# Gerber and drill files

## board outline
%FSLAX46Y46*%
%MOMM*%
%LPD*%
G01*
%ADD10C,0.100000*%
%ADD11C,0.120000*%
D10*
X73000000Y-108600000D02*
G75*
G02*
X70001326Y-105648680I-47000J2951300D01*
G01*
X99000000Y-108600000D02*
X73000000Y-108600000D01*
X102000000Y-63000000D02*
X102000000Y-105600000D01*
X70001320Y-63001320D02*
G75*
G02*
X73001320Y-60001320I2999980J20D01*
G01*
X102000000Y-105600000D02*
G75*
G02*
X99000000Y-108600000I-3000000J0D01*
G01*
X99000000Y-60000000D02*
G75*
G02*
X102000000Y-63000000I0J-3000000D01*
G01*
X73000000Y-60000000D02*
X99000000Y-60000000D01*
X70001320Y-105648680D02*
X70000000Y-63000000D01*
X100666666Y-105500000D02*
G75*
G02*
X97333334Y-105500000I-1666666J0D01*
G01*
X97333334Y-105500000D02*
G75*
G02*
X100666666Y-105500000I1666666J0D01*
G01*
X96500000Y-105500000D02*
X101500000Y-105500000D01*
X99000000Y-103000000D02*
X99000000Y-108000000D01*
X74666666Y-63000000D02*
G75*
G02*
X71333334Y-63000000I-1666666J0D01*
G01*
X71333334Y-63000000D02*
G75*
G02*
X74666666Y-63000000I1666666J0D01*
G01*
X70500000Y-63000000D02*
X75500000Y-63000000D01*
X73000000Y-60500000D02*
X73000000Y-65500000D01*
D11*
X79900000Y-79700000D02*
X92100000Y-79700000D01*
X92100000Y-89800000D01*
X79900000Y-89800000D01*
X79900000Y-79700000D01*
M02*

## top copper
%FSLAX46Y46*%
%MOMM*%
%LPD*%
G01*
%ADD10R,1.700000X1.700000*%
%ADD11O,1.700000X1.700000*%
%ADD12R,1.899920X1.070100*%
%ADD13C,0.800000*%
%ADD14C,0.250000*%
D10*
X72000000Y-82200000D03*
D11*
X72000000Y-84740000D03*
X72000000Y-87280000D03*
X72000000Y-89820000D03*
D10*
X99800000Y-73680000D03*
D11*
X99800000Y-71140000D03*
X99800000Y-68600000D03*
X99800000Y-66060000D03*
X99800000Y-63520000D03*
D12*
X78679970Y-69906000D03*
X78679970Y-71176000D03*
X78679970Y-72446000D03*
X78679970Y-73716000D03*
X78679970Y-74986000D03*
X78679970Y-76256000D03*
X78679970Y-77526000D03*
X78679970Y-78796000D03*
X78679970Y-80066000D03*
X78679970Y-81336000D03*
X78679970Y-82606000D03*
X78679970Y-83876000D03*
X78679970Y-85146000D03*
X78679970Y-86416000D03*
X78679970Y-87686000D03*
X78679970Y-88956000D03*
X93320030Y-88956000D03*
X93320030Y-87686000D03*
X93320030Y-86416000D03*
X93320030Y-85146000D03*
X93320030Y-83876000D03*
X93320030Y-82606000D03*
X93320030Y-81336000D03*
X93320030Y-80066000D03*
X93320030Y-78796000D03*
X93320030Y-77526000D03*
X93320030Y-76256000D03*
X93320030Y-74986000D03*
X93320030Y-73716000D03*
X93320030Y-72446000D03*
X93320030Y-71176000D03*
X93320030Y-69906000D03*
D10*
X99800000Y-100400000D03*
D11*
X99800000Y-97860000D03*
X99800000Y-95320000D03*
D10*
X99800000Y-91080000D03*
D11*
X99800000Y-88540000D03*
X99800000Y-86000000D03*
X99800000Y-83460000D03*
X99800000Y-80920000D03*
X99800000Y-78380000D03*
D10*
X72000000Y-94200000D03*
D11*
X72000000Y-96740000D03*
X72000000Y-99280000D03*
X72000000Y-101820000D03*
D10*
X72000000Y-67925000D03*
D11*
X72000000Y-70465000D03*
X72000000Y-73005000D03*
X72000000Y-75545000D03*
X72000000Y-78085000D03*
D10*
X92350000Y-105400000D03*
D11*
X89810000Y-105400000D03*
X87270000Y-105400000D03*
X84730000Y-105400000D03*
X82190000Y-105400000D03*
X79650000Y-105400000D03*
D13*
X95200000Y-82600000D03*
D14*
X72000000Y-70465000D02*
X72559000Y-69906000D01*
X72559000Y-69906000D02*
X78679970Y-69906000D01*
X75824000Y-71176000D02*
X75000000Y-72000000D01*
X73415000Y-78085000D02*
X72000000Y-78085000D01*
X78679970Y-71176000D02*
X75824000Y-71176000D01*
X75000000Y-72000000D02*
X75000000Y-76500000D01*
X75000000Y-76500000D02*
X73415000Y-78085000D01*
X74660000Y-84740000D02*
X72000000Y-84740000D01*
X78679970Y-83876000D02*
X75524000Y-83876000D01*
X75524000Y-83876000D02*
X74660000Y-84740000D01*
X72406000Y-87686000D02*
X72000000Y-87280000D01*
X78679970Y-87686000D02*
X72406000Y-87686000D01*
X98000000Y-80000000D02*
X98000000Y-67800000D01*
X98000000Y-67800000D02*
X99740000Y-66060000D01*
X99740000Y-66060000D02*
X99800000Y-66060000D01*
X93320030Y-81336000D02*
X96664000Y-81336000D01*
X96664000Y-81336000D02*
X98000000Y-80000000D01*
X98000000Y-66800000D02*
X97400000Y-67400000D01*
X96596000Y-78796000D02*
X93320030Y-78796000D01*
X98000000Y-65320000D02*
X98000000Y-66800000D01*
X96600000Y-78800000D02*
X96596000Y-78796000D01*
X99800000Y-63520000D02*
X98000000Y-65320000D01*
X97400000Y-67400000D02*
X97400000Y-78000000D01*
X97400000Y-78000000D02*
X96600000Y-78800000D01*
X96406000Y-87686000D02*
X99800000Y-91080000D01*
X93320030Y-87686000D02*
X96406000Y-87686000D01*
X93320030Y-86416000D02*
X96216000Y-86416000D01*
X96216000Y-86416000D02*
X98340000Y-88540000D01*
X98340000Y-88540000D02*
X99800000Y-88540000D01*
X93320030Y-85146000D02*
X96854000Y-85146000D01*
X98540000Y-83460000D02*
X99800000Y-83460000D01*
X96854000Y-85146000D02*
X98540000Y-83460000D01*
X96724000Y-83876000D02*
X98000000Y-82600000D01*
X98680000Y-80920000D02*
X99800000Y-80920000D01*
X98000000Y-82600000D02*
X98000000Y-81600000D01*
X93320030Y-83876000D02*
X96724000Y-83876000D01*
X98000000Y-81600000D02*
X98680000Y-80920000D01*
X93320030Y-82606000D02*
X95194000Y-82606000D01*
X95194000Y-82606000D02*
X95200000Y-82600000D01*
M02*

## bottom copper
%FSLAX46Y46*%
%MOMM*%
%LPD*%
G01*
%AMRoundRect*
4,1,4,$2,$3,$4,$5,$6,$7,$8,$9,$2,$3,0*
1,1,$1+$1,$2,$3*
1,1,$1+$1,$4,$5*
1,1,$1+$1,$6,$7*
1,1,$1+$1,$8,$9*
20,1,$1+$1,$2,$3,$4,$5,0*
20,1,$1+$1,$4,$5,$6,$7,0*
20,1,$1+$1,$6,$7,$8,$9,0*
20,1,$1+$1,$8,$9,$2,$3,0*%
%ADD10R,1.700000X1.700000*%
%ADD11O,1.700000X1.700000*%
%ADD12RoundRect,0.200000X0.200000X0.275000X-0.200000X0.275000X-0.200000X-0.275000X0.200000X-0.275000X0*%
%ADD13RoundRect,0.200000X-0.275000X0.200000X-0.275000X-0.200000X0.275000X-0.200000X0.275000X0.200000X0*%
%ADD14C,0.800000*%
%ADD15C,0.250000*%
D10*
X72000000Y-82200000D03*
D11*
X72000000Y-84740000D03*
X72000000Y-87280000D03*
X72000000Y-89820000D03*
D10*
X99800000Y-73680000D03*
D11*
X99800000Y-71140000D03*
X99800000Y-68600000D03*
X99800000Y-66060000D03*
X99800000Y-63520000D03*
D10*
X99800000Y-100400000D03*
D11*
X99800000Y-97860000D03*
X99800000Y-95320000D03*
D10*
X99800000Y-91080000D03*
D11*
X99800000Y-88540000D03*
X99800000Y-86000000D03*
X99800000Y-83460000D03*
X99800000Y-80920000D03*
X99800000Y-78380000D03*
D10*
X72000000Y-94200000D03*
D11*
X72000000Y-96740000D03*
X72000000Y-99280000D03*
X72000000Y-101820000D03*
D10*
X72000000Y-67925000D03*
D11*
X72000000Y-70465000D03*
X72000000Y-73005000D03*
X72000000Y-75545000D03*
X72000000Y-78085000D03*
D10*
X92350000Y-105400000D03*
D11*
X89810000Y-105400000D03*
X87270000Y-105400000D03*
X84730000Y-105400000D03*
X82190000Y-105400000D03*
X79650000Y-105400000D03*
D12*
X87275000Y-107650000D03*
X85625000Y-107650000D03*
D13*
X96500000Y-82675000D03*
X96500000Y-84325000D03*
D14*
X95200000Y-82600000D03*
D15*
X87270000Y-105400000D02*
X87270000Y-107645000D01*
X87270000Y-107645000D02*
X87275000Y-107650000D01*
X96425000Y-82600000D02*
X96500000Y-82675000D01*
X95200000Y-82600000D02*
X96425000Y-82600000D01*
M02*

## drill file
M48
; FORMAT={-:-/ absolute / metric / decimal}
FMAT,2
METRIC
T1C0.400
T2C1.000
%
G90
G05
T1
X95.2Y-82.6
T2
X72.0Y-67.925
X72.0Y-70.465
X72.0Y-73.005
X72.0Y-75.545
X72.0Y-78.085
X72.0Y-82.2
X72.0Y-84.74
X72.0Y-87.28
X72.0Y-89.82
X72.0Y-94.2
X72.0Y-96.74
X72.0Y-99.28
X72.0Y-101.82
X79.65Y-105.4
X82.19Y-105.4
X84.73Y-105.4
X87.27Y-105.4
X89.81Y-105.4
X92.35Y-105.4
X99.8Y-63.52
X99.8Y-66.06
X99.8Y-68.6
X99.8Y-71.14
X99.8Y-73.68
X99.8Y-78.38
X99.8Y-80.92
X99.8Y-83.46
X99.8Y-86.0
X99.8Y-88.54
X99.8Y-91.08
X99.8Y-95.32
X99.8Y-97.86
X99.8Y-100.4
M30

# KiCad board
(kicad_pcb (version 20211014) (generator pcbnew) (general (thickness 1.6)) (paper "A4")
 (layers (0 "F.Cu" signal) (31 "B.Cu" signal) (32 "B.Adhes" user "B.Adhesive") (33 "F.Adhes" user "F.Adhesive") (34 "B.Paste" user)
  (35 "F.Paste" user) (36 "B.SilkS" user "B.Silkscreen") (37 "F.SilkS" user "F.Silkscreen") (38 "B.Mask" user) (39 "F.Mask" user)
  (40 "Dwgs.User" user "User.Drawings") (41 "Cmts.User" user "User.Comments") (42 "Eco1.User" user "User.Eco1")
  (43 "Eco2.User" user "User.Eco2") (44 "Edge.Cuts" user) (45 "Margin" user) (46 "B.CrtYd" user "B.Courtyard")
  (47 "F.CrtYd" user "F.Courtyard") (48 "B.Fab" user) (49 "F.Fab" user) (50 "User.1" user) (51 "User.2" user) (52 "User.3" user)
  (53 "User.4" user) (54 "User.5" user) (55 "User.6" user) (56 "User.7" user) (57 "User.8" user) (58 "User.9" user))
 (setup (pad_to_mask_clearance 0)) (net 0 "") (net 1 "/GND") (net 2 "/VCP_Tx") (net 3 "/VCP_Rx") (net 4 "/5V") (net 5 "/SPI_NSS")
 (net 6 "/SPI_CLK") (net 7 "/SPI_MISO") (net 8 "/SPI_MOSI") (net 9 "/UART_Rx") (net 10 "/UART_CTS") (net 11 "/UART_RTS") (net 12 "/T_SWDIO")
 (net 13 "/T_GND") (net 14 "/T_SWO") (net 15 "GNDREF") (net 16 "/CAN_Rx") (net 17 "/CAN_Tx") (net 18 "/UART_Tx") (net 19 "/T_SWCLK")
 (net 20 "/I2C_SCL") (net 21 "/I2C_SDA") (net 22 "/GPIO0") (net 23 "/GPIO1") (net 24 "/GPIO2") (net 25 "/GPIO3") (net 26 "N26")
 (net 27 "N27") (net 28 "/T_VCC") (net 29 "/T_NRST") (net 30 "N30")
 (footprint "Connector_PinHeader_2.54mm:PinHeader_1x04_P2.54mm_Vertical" (layer "F.Cu") (at 72 82.2)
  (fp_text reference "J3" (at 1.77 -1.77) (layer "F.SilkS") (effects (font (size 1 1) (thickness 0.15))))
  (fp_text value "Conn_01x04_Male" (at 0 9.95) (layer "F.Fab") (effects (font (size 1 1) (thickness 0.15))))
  (pad "1" thru_hole rect (at 0 0) (size 1.7 1.7) (drill 1) (layers *.Cu *.Mask) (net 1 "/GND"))
  (pad "2" thru_hole oval (at 0 2.54) (size 1.7 1.7) (drill 1) (layers *.Cu *.Mask) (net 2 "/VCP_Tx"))
  (pad "3" thru_hole oval (at 0 5.08) (size 1.7 1.7) (drill 1) (layers *.Cu *.Mask) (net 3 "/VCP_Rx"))
  (pad "4" thru_hole oval (at 0 7.62) (size 1.7 1.7) (drill 1) (layers *.Cu *.Mask) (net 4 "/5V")))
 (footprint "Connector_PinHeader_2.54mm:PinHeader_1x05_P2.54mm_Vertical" (layer "F.Cu") (at 99.8 73.68 180)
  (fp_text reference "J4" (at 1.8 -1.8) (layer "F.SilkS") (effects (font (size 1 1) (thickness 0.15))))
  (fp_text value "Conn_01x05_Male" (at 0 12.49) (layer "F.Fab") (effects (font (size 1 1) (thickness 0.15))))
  (pad "1" thru_hole rect (at 0 0 180) (size 1.7 1.7) (drill 1) (layers *.Cu *.Mask) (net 1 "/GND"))
  (pad "2" thru_hole oval (at 0 2.54 180) (size 1.7 1.7) (drill 1) (layers *.Cu *.Mask) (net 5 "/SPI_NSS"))
  (pad "3" thru_hole oval (at 0 5.08 180) (size 1.7 1.7) (drill 1) (layers *.Cu *.Mask) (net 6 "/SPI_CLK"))
  (pad "4" thru_hole oval (at 0 7.62 180) (size 1.7 1.7) (drill 1) (layers *.Cu *.Mask) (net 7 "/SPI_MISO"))
  (pad "5" thru_hole oval (at 0 10.16 180) (size 1.7 1.7) (drill 1) (layers *.Cu *.Mask) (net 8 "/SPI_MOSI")))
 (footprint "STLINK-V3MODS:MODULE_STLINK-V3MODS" (layer "F.Cu") (at 86 60)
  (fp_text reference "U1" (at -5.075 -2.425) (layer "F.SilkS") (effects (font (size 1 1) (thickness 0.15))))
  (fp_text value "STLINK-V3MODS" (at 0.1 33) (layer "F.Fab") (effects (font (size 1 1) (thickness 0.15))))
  (fp_rect (start -6.1 19.7) (end 6.1 29.8) (layer "Edge.Cuts") (width 0.12) (fill none))
  (pad "1" smd rect (at -7.32003 9.906) (size 1.89992 1.0701) (layers "F.Cu" "F.Paste" "F.Mask") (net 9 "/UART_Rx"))
  (pad "2" smd rect (at -7.32003 11.176) (size 1.89992 1.0701) (layers "F.Cu" "F.Paste" "F.Mask") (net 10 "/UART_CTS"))
  (pad "3" smd rect (at -7.32003 12.446) (size 1.89992 1.0701) (layers "F.Cu" "F.Paste" "F.Mask") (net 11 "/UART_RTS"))
  (pad "4" smd rect (at -7.32003 13.716) (size 1.89992 1.0701) (layers "F.Cu" "F.Paste" "F.Mask") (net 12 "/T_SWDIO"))
  (pad "5" smd rect (at -7.32003 14.986) (size 1.89992 1.0701) (layers "F.Cu" "F.Paste" "F.Mask") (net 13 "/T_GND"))
  (pad "6" smd rect (at -7.32003 16.256) (size 1.89992 1.0701) (layers "F.Cu" "F.Paste" "F.Mask") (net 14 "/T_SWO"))
  (pad "7" smd rect (at -7.32003 17.526) (size 1.89992 1.0701) (layers "F.Cu" "F.Paste" "F.Mask") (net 6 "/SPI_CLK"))
  (pad "8" smd rect (at -7.32003 18.796) (size 1.89992 1.0701) (layers "F.Cu" "F.Paste" "F.Mask") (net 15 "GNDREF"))
  (pad "9" smd rect (at -7.32003 20.066) (size 1.89992 1.0701) (layers "F.Cu" "F.Paste" "F.Mask") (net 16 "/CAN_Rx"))
  (pad "10" smd rect (at -7.32003 21.336) (size 1.89992 1.0701) (layers "F.Cu" "F.Paste" "F.Mask") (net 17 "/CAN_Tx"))
  (pad "11" smd rect (at -7.32003 22.606) (size 1.89992 1.0701) (layers "F.Cu" "F.Paste" "F.Mask") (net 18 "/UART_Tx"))
  (pad "12" smd rect (at -7.32003 23.876) (size 1.89992 1.0701) (layers "F.Cu" "F.Paste" "F.Mask") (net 2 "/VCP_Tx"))
  (pad "13" smd rect (at -7.32003 25.146) (size 1.89992 1.0701) (layers "F.Cu" "F.Paste" "F.Mask") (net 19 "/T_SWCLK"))
  (pad "14" smd rect (at -7.32003 26.416) (size 1.89992 1.0701) (layers "F.Cu" "F.Paste" "F.Mask") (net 5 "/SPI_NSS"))
  (pad "15" smd rect (at -7.32003 27.686) (size 1.89992 1.0701) (layers "F.Cu" "F.Paste" "F.Mask") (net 3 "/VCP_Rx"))
  (pad "16" smd rect (at -7.32003 28.956) (size 1.89992 1.0701) (layers "F.Cu" "F.Paste" "F.Mask") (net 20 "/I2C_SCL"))
  (pad "17" smd rect (at 7.32003 28.956 180) (size 1.89992 1.0701) (layers "F.Cu" "F.Paste" "F.Mask") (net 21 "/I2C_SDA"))
  (pad "18" smd rect (at 7.32003 27.686 180) (size 1.89992 1.0701) (layers "F.Cu" "F.Paste" "F.Mask") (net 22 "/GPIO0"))
  (pad "19" smd rect (at 7.32003 26.416 180) (size 1.89992 1.0701) (layers "F.Cu" "F.Paste" "F.Mask") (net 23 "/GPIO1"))
  (pad "20" smd rect (at 7.32003 25.146 180) (size 1.89992 1.0701) (layers "F.Cu" "F.Paste" "F.Mask") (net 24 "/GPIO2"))
  (pad "21" smd rect (at 7.32003 23.876 180) (size 1.89992 1.0701) (layers "F.Cu" "F.Paste" "F.Mask") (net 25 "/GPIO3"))
  (pad "22" smd rect (at 7.32003 22.606 180) (size 1.89992 1.0701) (layers "F.Cu" "F.Paste" "F.Mask") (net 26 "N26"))
  (pad "23" smd rect (at 7.32003 21.336 180) (size 1.89992 1.0701) (layers "F.Cu" "F.Paste" "F.Mask") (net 7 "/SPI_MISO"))
  (pad "24" smd rect (at 7.32003 20.066 180) (size 1.89992 1.0701) (layers "F.Cu" "F.Paste" "F.Mask") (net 15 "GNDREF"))
  (pad "25" smd rect (at 7.32003 18.796 180) (size 1.89992 1.0701) (layers "F.Cu" "F.Paste" "F.Mask") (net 8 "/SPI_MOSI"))
  (pad "26" smd rect (at 7.32003 17.526 180) (size 1.89992 1.0701) (layers "F.Cu" "F.Paste" "F.Mask") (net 15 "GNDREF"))
  (pad "27" smd rect (at 7.32003 16.256 180) (size 1.89992 1.0701) (layers "F.Cu" "F.Paste" "F.Mask") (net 15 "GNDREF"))
  (pad "28" smd rect (at 7.32003 14.986 180) (size 1.89992 1.0701) (layers "F.Cu" "F.Paste" "F.Mask") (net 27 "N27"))
  (pad "29" smd rect (at 7.32003 13.716 180) (size 1.89992 1.0701) (layers "F.Cu" "F.Paste" "F.Mask") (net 15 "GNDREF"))
  (pad "30" smd rect (at 7.32003 12.446 180) (size 1.89992 1.0701) (layers "F.Cu" "F.Paste" "F.Mask") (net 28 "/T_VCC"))
  (pad "31" smd rect (at 7.32003 11.176 180) (size 1.89992 1.0701) (layers "F.Cu" "F.Paste" "F.Mask") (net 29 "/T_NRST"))
  (pad "32" smd rect (at 7.32003 9.906 180) (size 1.89992 1.0701) (layers "F.Cu" "F.Paste" "F.Mask") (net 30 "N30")))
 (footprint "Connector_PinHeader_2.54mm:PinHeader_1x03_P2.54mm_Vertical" (layer "F.Cu") (at 99.8 100.4 180)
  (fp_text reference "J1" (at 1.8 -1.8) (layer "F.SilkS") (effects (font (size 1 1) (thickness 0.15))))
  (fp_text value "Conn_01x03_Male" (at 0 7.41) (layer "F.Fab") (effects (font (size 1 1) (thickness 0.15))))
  (pad "1" thru_hole rect (at 0 0 180) (size 1.7 1.7) (drill 1) (layers *.Cu *.Mask) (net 1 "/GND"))
  (pad "2" thru_hole oval (at 0 2.54 180) (size 1.7 1.7) (drill 1) (layers *.Cu *.Mask) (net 21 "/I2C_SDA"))
  (pad "3" thru_hole oval (at 0 5.08 180) (size 1.7 1.7) (drill 1) (layers *.Cu *.Mask) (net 20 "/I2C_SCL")))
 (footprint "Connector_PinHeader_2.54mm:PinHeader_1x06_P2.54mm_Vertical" (layer "F.Cu") (at 99.8 91.08 180)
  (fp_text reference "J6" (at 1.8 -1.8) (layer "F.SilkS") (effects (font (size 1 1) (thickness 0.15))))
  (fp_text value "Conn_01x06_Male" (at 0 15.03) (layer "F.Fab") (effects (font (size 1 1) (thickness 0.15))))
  (pad "1" thru_hole rect (at 0 0 180) (size 1.7 1.7) (drill 1) (layers *.Cu *.Mask) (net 22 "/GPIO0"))
  (pad "2" thru_hole oval (at 0 2.54 180) (size 1.7 1.7) (drill 1) (layers *.Cu *.Mask) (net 23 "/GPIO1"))
  (pad "3" thru_hole oval (at 0 5.08 180) (size 1.7 1.7) (drill 1) (layers *.Cu *.Mask) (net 1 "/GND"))
  (pad "4" thru_hole oval (at 0 7.62 180) (size 1.7 1.7) (drill 1) (layers *.Cu *.Mask) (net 24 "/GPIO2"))
  (pad "5" thru_hole oval (at 0 10.16 180) (size 1.7 1.7) (drill 1) (layers *.Cu *.Mask) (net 25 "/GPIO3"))
  (pad "6" thru_hole oval (at 0 12.7 180) (size 1.7 1.7) (drill 1) (layers *.Cu *.Mask) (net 4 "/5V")))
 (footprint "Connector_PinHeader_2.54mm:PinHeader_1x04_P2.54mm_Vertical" (layer "F.Cu") (at 72 94.2)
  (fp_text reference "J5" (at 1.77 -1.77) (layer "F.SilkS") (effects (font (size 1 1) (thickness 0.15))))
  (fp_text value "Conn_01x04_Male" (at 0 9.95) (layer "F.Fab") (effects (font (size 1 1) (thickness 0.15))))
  (pad "1" thru_hole rect (at 0 0) (size 1.7 1.7) (drill 1) (layers *.Cu *.Mask) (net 1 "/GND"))
  (pad "2" thru_hole oval (at 0 2.54) (size 1.7 1.7) (drill 1) (layers *.Cu *.Mask) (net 17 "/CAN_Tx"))
  (pad "3" thru_hole oval (at 0 5.08) (size 1.7 1.7) (drill 1) (layers *.Cu *.Mask) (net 4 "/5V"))
  (pad "4" thru_hole oval (at 0 7.62) (size 1.7 1.7) (drill 1) (layers *.Cu *.Mask) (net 16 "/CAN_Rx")))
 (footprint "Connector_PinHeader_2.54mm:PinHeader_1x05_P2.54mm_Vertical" (layer "F.Cu") (at 72 67.925)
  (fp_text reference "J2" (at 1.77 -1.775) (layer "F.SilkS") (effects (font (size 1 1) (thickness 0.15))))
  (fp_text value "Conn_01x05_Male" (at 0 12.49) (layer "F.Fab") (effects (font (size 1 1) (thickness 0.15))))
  (pad "1" thru_hole rect (at 0 0) (size 1.7 1.7) (drill 1) (layers *.Cu *.Mask) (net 1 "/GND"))
  (pad "2" thru_hole oval (at 0 2.54) (size 1.7 1.7) (drill 1) (layers *.Cu *.Mask) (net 9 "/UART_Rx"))
  (pad "3" thru_hole oval (at 0 5.08) (size 1.7 1.7) (drill 1) (layers *.Cu *.Mask) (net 18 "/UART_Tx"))
  (pad "4" thru_hole oval (at 0 7.62) (size 1.7 1.7) (drill 1) (layers *.Cu *.Mask) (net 11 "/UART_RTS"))
  (pad "5" thru_hole oval (at 0 10.16) (size 1.7 1.7) (drill 1) (layers *.Cu *.Mask) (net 10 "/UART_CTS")))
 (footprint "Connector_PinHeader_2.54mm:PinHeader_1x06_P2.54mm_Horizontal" (layer "F.Cu") (at 92.35 105.4 -90)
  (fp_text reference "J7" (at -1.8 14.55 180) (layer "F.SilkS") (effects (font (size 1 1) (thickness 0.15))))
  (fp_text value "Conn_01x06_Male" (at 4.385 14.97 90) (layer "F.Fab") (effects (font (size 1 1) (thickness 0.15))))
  (pad "1" thru_hole rect (at 0 0 270) (size 1.7 1.7) (drill 1) (layers *.Cu *.Mask) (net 28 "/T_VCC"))
  (pad "2" thru_hole oval (at 0 2.54 270) (size 1.7 1.7) (drill 1) (layers *.Cu *.Mask) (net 19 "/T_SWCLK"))
  (pad "3" thru_hole oval (at 0 5.08 270) (size 1.7 1.7) (drill 1) (layers *.Cu *.Mask) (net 13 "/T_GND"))
  (pad "4" thru_hole oval (at 0 7.62 270) (size 1.7 1.7) (drill 1) (layers *.Cu *.Mask) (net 12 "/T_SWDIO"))
  (pad "5" thru_hole oval (at 0 10.16 270) (size 1.7 1.7) (drill 1) (layers *.Cu *.Mask) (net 29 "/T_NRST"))
  (pad "6" thru_hole oval (at 0 12.7 270) (size 1.7 1.7) (drill 1) (layers *.Cu *.Mask) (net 14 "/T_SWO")))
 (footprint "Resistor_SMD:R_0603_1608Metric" (layer "B.Cu") (at 86.45 107.65 180)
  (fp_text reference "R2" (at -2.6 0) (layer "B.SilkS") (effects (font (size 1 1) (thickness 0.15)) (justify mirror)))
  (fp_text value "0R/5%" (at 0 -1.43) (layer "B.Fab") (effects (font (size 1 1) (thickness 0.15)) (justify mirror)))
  (pad "1" smd roundrect (at -0.825 0 180) (size 0.8 0.95) (layers "B.Cu" "B.Paste" "B.Mask") (roundrect_rratio 0.25) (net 13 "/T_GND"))
  (pad "2" smd roundrect (at 0.825 0 180) (size 0.8 0.95) (layers "B.Cu" "B.Paste" "B.Mask") (roundrect_rratio 0.25) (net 15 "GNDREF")))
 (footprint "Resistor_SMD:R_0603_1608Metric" (layer "B.Cu") (at 96.5 83.5 -90)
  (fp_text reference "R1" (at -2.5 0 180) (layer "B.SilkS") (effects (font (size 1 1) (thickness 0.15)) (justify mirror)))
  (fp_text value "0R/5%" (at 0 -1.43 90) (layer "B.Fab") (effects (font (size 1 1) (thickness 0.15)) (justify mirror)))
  (pad "1" smd roundrect (at -0.825 0 270) (size 0.8 0.95) (layers "B.Cu" "B.Paste" "B.Mask") (roundrect_rratio 0.25) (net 26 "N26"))
  (pad "2" smd roundrect (at 0.825 0 270) (size 0.8 0.95) (layers "B.Cu" "B.Paste" "B.Mask") (roundrect_rratio 0.25) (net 4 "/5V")))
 (gr_arc (start 73 108.6) (mid 70.882523 107.752395) (end 70.00132 105.64868) (layer "Edge.Cuts") (width 0.1))
 (gr_line (start 99 108.6) (end 73 108.6) (layer "Edge.Cuts") (width 0.1))
 (gr_line (start 102 63) (end 102 105.6) (layer "Edge.Cuts") (width 0.1))
 (gr_arc (start 70.00132 63.00132) (mid 70.88 60.88) (end 73.00132 60.00132) (layer "Edge.Cuts") (width 0.1))
 (gr_arc (start 102 105.6) (mid 101.121326 107.721326) (end 99 108.6) (layer "Edge.Cuts") (width 0.1))
 (gr_arc (start 99 60) (mid 101.12132 60.87868) (end 102 63) (layer "Edge.Cuts") (width 0.1))
 (gr_line (start 73 60) (end 99 60) (layer "Edge.Cuts") (width 0.1))
 (gr_line (start 70.00132 105.64868) (end 70 63) (layer "Edge.Cuts") (width 0.1))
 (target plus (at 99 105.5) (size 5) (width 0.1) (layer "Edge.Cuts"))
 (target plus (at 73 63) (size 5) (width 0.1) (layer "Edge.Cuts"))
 (segment (start 72 70.465) (end 72.559 69.906) (width 0.25) (layer "F.Cu") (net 9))
 (segment (start 72.559 69.906) (end 78.67997 69.906) (width 0.25) (layer "F.Cu") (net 9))
 (segment (start 75.824 71.176) (end 75 72) (width 0.25) (layer "F.Cu") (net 10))
 (segment (start 73.415 78.085) (end 72 78.085) (width 0.25) (layer "F.Cu") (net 10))
 (segment (start 78.67997 71.176) (end 75.824 71.176) (width 0.25) (layer "F.Cu") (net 10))
 (segment (start 75 72) (end 75 76.5) (width 0.25) (layer "F.Cu") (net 10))
 (segment (start 75 76.5) (end 73.415 78.085) (width 0.25) (layer "F.Cu") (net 10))
 (segment (start 74.66 84.74) (end 72 84.74) (width 0.25) (layer "F.Cu") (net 2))
 (segment (start 78.67997 83.876) (end 75.524 83.876) (width 0.25) (layer "F.Cu") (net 2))
 (segment (start 75.524 83.876) (end 74.66 84.74) (width 0.25) (layer "F.Cu") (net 2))
 (segment (start 72.406 87.686) (end 72 87.28) (width 0.25) (layer "F.Cu") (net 3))
 (segment (start 78.67997 87.686) (end 72.406 87.686) (width 0.25) (layer "F.Cu") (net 3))
 (segment (start 98 80) (end 98 67.8) (width 0.25) (layer "F.Cu") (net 7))
 (segment (start 98 67.8) (end 99.74 66.06) (width 0.25) (layer "F.Cu") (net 7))
 (segment (start 99.74 66.06) (end 99.8 66.06) (width 0.25) (layer "F.Cu") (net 7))
 (segment (start 93.32003 81.336) (end 96.664 81.336) (width 0.25) (layer "F.Cu") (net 7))
 (segment (start 96.664 81.336) (end 98 80) (width 0.25) (layer "F.Cu") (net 7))
 (segment (start 98 66.8) (end 97.4 67.4) (width 0.25) (layer "F.Cu") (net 8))
 (segment (start 96.596 78.796) (end 93.32003 78.796) (width 0.25) (layer "F.Cu") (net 8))
 (segment (start 98 65.32) (end 98 66.8) (width 0.25) (layer "F.Cu") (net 8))
 (segment (start 96.6 78.8) (end 96.596 78.796) (width 0.25) (layer "F.Cu") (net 8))
 (segment (start 99.8 63.52) (end 98 65.32) (width 0.25) (layer "F.Cu") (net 8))
 (segment (start 97.4 67.4) (end 97.4 78) (width 0.25) (layer "F.Cu") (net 8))
 (segment (start 97.4 78) (end 96.6 78.8) (width 0.25) (layer "F.Cu") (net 8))
 (segment (start 96.406 87.686) (end 99.8 91.08) (width 0.25) (layer "F.Cu") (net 22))
 (segment (start 93.32003 87.686) (end 96.406 87.686) (width 0.25) (layer "F.Cu") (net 22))
 (segment (start 93.32003 86.416) (end 96.216 86.416) (width 0.25) (layer "F.Cu") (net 23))
 (segment (start 96.216 86.416) (end 98.34 88.54) (width 0.25) (layer "F.Cu") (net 23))
 (segment (start 98.34 88.54) (end 99.8 88.54) (width 0.25) (layer "F.Cu") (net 23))
 (segment (start 93.32003 85.146) (end 96.854 85.146) (width 0.25) (layer "F.Cu") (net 24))
 (segment (start 98.54 83.46) (end 99.8 83.46) (width 0.25) (layer "F.Cu") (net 24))
 (segment (start 96.854 85.146) (end 98.54 83.46) (width 0.25) (layer "F.Cu") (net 24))
 (segment (start 96.724 83.876) (end 98 82.6) (width 0.25) (layer "F.Cu") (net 25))
 (segment (start 98.68 80.92) (end 99.8 80.92) (width 0.25) (layer "F.Cu") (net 25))
 (segment (start 98 82.6) (end 98 81.6) (width 0.25) (layer "F.Cu") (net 25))
 (segment (start 93.32003 83.876) (end 96.724 83.876) (width 0.25) (layer "F.Cu") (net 25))
 (segment (start 98 81.6) (end 98.68 80.92) (width 0.25) (layer "F.Cu") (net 25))
 (segment (start 87.27 105.4) (end 87.27 107.645) (width 0.25) (layer "B.Cu") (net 13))
 (segment (start 87.27 107.645) (end 87.275 107.65) (width 0.25) (layer "B.Cu") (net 13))
 (segment (start 93.32003 82.606) (end 95.194 82.606) (width 0.25) (layer "F.Cu") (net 26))
 (segment (start 95.194 82.606) (end 95.2 82.6) (width 0.25) (layer "F.Cu") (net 26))
 (via (at 95.2 82.6) (size 0.8) (drill 0.4) (layers "F.Cu" "B.Cu") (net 26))
 (segment (start 96.425 82.6) (end 96.5 82.675) (width 0.25) (layer "B.Cu") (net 26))
 (segment (start 95.2 82.6) (end 96.425 82.6) (width 0.25) (layer "B.Cu") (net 26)))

